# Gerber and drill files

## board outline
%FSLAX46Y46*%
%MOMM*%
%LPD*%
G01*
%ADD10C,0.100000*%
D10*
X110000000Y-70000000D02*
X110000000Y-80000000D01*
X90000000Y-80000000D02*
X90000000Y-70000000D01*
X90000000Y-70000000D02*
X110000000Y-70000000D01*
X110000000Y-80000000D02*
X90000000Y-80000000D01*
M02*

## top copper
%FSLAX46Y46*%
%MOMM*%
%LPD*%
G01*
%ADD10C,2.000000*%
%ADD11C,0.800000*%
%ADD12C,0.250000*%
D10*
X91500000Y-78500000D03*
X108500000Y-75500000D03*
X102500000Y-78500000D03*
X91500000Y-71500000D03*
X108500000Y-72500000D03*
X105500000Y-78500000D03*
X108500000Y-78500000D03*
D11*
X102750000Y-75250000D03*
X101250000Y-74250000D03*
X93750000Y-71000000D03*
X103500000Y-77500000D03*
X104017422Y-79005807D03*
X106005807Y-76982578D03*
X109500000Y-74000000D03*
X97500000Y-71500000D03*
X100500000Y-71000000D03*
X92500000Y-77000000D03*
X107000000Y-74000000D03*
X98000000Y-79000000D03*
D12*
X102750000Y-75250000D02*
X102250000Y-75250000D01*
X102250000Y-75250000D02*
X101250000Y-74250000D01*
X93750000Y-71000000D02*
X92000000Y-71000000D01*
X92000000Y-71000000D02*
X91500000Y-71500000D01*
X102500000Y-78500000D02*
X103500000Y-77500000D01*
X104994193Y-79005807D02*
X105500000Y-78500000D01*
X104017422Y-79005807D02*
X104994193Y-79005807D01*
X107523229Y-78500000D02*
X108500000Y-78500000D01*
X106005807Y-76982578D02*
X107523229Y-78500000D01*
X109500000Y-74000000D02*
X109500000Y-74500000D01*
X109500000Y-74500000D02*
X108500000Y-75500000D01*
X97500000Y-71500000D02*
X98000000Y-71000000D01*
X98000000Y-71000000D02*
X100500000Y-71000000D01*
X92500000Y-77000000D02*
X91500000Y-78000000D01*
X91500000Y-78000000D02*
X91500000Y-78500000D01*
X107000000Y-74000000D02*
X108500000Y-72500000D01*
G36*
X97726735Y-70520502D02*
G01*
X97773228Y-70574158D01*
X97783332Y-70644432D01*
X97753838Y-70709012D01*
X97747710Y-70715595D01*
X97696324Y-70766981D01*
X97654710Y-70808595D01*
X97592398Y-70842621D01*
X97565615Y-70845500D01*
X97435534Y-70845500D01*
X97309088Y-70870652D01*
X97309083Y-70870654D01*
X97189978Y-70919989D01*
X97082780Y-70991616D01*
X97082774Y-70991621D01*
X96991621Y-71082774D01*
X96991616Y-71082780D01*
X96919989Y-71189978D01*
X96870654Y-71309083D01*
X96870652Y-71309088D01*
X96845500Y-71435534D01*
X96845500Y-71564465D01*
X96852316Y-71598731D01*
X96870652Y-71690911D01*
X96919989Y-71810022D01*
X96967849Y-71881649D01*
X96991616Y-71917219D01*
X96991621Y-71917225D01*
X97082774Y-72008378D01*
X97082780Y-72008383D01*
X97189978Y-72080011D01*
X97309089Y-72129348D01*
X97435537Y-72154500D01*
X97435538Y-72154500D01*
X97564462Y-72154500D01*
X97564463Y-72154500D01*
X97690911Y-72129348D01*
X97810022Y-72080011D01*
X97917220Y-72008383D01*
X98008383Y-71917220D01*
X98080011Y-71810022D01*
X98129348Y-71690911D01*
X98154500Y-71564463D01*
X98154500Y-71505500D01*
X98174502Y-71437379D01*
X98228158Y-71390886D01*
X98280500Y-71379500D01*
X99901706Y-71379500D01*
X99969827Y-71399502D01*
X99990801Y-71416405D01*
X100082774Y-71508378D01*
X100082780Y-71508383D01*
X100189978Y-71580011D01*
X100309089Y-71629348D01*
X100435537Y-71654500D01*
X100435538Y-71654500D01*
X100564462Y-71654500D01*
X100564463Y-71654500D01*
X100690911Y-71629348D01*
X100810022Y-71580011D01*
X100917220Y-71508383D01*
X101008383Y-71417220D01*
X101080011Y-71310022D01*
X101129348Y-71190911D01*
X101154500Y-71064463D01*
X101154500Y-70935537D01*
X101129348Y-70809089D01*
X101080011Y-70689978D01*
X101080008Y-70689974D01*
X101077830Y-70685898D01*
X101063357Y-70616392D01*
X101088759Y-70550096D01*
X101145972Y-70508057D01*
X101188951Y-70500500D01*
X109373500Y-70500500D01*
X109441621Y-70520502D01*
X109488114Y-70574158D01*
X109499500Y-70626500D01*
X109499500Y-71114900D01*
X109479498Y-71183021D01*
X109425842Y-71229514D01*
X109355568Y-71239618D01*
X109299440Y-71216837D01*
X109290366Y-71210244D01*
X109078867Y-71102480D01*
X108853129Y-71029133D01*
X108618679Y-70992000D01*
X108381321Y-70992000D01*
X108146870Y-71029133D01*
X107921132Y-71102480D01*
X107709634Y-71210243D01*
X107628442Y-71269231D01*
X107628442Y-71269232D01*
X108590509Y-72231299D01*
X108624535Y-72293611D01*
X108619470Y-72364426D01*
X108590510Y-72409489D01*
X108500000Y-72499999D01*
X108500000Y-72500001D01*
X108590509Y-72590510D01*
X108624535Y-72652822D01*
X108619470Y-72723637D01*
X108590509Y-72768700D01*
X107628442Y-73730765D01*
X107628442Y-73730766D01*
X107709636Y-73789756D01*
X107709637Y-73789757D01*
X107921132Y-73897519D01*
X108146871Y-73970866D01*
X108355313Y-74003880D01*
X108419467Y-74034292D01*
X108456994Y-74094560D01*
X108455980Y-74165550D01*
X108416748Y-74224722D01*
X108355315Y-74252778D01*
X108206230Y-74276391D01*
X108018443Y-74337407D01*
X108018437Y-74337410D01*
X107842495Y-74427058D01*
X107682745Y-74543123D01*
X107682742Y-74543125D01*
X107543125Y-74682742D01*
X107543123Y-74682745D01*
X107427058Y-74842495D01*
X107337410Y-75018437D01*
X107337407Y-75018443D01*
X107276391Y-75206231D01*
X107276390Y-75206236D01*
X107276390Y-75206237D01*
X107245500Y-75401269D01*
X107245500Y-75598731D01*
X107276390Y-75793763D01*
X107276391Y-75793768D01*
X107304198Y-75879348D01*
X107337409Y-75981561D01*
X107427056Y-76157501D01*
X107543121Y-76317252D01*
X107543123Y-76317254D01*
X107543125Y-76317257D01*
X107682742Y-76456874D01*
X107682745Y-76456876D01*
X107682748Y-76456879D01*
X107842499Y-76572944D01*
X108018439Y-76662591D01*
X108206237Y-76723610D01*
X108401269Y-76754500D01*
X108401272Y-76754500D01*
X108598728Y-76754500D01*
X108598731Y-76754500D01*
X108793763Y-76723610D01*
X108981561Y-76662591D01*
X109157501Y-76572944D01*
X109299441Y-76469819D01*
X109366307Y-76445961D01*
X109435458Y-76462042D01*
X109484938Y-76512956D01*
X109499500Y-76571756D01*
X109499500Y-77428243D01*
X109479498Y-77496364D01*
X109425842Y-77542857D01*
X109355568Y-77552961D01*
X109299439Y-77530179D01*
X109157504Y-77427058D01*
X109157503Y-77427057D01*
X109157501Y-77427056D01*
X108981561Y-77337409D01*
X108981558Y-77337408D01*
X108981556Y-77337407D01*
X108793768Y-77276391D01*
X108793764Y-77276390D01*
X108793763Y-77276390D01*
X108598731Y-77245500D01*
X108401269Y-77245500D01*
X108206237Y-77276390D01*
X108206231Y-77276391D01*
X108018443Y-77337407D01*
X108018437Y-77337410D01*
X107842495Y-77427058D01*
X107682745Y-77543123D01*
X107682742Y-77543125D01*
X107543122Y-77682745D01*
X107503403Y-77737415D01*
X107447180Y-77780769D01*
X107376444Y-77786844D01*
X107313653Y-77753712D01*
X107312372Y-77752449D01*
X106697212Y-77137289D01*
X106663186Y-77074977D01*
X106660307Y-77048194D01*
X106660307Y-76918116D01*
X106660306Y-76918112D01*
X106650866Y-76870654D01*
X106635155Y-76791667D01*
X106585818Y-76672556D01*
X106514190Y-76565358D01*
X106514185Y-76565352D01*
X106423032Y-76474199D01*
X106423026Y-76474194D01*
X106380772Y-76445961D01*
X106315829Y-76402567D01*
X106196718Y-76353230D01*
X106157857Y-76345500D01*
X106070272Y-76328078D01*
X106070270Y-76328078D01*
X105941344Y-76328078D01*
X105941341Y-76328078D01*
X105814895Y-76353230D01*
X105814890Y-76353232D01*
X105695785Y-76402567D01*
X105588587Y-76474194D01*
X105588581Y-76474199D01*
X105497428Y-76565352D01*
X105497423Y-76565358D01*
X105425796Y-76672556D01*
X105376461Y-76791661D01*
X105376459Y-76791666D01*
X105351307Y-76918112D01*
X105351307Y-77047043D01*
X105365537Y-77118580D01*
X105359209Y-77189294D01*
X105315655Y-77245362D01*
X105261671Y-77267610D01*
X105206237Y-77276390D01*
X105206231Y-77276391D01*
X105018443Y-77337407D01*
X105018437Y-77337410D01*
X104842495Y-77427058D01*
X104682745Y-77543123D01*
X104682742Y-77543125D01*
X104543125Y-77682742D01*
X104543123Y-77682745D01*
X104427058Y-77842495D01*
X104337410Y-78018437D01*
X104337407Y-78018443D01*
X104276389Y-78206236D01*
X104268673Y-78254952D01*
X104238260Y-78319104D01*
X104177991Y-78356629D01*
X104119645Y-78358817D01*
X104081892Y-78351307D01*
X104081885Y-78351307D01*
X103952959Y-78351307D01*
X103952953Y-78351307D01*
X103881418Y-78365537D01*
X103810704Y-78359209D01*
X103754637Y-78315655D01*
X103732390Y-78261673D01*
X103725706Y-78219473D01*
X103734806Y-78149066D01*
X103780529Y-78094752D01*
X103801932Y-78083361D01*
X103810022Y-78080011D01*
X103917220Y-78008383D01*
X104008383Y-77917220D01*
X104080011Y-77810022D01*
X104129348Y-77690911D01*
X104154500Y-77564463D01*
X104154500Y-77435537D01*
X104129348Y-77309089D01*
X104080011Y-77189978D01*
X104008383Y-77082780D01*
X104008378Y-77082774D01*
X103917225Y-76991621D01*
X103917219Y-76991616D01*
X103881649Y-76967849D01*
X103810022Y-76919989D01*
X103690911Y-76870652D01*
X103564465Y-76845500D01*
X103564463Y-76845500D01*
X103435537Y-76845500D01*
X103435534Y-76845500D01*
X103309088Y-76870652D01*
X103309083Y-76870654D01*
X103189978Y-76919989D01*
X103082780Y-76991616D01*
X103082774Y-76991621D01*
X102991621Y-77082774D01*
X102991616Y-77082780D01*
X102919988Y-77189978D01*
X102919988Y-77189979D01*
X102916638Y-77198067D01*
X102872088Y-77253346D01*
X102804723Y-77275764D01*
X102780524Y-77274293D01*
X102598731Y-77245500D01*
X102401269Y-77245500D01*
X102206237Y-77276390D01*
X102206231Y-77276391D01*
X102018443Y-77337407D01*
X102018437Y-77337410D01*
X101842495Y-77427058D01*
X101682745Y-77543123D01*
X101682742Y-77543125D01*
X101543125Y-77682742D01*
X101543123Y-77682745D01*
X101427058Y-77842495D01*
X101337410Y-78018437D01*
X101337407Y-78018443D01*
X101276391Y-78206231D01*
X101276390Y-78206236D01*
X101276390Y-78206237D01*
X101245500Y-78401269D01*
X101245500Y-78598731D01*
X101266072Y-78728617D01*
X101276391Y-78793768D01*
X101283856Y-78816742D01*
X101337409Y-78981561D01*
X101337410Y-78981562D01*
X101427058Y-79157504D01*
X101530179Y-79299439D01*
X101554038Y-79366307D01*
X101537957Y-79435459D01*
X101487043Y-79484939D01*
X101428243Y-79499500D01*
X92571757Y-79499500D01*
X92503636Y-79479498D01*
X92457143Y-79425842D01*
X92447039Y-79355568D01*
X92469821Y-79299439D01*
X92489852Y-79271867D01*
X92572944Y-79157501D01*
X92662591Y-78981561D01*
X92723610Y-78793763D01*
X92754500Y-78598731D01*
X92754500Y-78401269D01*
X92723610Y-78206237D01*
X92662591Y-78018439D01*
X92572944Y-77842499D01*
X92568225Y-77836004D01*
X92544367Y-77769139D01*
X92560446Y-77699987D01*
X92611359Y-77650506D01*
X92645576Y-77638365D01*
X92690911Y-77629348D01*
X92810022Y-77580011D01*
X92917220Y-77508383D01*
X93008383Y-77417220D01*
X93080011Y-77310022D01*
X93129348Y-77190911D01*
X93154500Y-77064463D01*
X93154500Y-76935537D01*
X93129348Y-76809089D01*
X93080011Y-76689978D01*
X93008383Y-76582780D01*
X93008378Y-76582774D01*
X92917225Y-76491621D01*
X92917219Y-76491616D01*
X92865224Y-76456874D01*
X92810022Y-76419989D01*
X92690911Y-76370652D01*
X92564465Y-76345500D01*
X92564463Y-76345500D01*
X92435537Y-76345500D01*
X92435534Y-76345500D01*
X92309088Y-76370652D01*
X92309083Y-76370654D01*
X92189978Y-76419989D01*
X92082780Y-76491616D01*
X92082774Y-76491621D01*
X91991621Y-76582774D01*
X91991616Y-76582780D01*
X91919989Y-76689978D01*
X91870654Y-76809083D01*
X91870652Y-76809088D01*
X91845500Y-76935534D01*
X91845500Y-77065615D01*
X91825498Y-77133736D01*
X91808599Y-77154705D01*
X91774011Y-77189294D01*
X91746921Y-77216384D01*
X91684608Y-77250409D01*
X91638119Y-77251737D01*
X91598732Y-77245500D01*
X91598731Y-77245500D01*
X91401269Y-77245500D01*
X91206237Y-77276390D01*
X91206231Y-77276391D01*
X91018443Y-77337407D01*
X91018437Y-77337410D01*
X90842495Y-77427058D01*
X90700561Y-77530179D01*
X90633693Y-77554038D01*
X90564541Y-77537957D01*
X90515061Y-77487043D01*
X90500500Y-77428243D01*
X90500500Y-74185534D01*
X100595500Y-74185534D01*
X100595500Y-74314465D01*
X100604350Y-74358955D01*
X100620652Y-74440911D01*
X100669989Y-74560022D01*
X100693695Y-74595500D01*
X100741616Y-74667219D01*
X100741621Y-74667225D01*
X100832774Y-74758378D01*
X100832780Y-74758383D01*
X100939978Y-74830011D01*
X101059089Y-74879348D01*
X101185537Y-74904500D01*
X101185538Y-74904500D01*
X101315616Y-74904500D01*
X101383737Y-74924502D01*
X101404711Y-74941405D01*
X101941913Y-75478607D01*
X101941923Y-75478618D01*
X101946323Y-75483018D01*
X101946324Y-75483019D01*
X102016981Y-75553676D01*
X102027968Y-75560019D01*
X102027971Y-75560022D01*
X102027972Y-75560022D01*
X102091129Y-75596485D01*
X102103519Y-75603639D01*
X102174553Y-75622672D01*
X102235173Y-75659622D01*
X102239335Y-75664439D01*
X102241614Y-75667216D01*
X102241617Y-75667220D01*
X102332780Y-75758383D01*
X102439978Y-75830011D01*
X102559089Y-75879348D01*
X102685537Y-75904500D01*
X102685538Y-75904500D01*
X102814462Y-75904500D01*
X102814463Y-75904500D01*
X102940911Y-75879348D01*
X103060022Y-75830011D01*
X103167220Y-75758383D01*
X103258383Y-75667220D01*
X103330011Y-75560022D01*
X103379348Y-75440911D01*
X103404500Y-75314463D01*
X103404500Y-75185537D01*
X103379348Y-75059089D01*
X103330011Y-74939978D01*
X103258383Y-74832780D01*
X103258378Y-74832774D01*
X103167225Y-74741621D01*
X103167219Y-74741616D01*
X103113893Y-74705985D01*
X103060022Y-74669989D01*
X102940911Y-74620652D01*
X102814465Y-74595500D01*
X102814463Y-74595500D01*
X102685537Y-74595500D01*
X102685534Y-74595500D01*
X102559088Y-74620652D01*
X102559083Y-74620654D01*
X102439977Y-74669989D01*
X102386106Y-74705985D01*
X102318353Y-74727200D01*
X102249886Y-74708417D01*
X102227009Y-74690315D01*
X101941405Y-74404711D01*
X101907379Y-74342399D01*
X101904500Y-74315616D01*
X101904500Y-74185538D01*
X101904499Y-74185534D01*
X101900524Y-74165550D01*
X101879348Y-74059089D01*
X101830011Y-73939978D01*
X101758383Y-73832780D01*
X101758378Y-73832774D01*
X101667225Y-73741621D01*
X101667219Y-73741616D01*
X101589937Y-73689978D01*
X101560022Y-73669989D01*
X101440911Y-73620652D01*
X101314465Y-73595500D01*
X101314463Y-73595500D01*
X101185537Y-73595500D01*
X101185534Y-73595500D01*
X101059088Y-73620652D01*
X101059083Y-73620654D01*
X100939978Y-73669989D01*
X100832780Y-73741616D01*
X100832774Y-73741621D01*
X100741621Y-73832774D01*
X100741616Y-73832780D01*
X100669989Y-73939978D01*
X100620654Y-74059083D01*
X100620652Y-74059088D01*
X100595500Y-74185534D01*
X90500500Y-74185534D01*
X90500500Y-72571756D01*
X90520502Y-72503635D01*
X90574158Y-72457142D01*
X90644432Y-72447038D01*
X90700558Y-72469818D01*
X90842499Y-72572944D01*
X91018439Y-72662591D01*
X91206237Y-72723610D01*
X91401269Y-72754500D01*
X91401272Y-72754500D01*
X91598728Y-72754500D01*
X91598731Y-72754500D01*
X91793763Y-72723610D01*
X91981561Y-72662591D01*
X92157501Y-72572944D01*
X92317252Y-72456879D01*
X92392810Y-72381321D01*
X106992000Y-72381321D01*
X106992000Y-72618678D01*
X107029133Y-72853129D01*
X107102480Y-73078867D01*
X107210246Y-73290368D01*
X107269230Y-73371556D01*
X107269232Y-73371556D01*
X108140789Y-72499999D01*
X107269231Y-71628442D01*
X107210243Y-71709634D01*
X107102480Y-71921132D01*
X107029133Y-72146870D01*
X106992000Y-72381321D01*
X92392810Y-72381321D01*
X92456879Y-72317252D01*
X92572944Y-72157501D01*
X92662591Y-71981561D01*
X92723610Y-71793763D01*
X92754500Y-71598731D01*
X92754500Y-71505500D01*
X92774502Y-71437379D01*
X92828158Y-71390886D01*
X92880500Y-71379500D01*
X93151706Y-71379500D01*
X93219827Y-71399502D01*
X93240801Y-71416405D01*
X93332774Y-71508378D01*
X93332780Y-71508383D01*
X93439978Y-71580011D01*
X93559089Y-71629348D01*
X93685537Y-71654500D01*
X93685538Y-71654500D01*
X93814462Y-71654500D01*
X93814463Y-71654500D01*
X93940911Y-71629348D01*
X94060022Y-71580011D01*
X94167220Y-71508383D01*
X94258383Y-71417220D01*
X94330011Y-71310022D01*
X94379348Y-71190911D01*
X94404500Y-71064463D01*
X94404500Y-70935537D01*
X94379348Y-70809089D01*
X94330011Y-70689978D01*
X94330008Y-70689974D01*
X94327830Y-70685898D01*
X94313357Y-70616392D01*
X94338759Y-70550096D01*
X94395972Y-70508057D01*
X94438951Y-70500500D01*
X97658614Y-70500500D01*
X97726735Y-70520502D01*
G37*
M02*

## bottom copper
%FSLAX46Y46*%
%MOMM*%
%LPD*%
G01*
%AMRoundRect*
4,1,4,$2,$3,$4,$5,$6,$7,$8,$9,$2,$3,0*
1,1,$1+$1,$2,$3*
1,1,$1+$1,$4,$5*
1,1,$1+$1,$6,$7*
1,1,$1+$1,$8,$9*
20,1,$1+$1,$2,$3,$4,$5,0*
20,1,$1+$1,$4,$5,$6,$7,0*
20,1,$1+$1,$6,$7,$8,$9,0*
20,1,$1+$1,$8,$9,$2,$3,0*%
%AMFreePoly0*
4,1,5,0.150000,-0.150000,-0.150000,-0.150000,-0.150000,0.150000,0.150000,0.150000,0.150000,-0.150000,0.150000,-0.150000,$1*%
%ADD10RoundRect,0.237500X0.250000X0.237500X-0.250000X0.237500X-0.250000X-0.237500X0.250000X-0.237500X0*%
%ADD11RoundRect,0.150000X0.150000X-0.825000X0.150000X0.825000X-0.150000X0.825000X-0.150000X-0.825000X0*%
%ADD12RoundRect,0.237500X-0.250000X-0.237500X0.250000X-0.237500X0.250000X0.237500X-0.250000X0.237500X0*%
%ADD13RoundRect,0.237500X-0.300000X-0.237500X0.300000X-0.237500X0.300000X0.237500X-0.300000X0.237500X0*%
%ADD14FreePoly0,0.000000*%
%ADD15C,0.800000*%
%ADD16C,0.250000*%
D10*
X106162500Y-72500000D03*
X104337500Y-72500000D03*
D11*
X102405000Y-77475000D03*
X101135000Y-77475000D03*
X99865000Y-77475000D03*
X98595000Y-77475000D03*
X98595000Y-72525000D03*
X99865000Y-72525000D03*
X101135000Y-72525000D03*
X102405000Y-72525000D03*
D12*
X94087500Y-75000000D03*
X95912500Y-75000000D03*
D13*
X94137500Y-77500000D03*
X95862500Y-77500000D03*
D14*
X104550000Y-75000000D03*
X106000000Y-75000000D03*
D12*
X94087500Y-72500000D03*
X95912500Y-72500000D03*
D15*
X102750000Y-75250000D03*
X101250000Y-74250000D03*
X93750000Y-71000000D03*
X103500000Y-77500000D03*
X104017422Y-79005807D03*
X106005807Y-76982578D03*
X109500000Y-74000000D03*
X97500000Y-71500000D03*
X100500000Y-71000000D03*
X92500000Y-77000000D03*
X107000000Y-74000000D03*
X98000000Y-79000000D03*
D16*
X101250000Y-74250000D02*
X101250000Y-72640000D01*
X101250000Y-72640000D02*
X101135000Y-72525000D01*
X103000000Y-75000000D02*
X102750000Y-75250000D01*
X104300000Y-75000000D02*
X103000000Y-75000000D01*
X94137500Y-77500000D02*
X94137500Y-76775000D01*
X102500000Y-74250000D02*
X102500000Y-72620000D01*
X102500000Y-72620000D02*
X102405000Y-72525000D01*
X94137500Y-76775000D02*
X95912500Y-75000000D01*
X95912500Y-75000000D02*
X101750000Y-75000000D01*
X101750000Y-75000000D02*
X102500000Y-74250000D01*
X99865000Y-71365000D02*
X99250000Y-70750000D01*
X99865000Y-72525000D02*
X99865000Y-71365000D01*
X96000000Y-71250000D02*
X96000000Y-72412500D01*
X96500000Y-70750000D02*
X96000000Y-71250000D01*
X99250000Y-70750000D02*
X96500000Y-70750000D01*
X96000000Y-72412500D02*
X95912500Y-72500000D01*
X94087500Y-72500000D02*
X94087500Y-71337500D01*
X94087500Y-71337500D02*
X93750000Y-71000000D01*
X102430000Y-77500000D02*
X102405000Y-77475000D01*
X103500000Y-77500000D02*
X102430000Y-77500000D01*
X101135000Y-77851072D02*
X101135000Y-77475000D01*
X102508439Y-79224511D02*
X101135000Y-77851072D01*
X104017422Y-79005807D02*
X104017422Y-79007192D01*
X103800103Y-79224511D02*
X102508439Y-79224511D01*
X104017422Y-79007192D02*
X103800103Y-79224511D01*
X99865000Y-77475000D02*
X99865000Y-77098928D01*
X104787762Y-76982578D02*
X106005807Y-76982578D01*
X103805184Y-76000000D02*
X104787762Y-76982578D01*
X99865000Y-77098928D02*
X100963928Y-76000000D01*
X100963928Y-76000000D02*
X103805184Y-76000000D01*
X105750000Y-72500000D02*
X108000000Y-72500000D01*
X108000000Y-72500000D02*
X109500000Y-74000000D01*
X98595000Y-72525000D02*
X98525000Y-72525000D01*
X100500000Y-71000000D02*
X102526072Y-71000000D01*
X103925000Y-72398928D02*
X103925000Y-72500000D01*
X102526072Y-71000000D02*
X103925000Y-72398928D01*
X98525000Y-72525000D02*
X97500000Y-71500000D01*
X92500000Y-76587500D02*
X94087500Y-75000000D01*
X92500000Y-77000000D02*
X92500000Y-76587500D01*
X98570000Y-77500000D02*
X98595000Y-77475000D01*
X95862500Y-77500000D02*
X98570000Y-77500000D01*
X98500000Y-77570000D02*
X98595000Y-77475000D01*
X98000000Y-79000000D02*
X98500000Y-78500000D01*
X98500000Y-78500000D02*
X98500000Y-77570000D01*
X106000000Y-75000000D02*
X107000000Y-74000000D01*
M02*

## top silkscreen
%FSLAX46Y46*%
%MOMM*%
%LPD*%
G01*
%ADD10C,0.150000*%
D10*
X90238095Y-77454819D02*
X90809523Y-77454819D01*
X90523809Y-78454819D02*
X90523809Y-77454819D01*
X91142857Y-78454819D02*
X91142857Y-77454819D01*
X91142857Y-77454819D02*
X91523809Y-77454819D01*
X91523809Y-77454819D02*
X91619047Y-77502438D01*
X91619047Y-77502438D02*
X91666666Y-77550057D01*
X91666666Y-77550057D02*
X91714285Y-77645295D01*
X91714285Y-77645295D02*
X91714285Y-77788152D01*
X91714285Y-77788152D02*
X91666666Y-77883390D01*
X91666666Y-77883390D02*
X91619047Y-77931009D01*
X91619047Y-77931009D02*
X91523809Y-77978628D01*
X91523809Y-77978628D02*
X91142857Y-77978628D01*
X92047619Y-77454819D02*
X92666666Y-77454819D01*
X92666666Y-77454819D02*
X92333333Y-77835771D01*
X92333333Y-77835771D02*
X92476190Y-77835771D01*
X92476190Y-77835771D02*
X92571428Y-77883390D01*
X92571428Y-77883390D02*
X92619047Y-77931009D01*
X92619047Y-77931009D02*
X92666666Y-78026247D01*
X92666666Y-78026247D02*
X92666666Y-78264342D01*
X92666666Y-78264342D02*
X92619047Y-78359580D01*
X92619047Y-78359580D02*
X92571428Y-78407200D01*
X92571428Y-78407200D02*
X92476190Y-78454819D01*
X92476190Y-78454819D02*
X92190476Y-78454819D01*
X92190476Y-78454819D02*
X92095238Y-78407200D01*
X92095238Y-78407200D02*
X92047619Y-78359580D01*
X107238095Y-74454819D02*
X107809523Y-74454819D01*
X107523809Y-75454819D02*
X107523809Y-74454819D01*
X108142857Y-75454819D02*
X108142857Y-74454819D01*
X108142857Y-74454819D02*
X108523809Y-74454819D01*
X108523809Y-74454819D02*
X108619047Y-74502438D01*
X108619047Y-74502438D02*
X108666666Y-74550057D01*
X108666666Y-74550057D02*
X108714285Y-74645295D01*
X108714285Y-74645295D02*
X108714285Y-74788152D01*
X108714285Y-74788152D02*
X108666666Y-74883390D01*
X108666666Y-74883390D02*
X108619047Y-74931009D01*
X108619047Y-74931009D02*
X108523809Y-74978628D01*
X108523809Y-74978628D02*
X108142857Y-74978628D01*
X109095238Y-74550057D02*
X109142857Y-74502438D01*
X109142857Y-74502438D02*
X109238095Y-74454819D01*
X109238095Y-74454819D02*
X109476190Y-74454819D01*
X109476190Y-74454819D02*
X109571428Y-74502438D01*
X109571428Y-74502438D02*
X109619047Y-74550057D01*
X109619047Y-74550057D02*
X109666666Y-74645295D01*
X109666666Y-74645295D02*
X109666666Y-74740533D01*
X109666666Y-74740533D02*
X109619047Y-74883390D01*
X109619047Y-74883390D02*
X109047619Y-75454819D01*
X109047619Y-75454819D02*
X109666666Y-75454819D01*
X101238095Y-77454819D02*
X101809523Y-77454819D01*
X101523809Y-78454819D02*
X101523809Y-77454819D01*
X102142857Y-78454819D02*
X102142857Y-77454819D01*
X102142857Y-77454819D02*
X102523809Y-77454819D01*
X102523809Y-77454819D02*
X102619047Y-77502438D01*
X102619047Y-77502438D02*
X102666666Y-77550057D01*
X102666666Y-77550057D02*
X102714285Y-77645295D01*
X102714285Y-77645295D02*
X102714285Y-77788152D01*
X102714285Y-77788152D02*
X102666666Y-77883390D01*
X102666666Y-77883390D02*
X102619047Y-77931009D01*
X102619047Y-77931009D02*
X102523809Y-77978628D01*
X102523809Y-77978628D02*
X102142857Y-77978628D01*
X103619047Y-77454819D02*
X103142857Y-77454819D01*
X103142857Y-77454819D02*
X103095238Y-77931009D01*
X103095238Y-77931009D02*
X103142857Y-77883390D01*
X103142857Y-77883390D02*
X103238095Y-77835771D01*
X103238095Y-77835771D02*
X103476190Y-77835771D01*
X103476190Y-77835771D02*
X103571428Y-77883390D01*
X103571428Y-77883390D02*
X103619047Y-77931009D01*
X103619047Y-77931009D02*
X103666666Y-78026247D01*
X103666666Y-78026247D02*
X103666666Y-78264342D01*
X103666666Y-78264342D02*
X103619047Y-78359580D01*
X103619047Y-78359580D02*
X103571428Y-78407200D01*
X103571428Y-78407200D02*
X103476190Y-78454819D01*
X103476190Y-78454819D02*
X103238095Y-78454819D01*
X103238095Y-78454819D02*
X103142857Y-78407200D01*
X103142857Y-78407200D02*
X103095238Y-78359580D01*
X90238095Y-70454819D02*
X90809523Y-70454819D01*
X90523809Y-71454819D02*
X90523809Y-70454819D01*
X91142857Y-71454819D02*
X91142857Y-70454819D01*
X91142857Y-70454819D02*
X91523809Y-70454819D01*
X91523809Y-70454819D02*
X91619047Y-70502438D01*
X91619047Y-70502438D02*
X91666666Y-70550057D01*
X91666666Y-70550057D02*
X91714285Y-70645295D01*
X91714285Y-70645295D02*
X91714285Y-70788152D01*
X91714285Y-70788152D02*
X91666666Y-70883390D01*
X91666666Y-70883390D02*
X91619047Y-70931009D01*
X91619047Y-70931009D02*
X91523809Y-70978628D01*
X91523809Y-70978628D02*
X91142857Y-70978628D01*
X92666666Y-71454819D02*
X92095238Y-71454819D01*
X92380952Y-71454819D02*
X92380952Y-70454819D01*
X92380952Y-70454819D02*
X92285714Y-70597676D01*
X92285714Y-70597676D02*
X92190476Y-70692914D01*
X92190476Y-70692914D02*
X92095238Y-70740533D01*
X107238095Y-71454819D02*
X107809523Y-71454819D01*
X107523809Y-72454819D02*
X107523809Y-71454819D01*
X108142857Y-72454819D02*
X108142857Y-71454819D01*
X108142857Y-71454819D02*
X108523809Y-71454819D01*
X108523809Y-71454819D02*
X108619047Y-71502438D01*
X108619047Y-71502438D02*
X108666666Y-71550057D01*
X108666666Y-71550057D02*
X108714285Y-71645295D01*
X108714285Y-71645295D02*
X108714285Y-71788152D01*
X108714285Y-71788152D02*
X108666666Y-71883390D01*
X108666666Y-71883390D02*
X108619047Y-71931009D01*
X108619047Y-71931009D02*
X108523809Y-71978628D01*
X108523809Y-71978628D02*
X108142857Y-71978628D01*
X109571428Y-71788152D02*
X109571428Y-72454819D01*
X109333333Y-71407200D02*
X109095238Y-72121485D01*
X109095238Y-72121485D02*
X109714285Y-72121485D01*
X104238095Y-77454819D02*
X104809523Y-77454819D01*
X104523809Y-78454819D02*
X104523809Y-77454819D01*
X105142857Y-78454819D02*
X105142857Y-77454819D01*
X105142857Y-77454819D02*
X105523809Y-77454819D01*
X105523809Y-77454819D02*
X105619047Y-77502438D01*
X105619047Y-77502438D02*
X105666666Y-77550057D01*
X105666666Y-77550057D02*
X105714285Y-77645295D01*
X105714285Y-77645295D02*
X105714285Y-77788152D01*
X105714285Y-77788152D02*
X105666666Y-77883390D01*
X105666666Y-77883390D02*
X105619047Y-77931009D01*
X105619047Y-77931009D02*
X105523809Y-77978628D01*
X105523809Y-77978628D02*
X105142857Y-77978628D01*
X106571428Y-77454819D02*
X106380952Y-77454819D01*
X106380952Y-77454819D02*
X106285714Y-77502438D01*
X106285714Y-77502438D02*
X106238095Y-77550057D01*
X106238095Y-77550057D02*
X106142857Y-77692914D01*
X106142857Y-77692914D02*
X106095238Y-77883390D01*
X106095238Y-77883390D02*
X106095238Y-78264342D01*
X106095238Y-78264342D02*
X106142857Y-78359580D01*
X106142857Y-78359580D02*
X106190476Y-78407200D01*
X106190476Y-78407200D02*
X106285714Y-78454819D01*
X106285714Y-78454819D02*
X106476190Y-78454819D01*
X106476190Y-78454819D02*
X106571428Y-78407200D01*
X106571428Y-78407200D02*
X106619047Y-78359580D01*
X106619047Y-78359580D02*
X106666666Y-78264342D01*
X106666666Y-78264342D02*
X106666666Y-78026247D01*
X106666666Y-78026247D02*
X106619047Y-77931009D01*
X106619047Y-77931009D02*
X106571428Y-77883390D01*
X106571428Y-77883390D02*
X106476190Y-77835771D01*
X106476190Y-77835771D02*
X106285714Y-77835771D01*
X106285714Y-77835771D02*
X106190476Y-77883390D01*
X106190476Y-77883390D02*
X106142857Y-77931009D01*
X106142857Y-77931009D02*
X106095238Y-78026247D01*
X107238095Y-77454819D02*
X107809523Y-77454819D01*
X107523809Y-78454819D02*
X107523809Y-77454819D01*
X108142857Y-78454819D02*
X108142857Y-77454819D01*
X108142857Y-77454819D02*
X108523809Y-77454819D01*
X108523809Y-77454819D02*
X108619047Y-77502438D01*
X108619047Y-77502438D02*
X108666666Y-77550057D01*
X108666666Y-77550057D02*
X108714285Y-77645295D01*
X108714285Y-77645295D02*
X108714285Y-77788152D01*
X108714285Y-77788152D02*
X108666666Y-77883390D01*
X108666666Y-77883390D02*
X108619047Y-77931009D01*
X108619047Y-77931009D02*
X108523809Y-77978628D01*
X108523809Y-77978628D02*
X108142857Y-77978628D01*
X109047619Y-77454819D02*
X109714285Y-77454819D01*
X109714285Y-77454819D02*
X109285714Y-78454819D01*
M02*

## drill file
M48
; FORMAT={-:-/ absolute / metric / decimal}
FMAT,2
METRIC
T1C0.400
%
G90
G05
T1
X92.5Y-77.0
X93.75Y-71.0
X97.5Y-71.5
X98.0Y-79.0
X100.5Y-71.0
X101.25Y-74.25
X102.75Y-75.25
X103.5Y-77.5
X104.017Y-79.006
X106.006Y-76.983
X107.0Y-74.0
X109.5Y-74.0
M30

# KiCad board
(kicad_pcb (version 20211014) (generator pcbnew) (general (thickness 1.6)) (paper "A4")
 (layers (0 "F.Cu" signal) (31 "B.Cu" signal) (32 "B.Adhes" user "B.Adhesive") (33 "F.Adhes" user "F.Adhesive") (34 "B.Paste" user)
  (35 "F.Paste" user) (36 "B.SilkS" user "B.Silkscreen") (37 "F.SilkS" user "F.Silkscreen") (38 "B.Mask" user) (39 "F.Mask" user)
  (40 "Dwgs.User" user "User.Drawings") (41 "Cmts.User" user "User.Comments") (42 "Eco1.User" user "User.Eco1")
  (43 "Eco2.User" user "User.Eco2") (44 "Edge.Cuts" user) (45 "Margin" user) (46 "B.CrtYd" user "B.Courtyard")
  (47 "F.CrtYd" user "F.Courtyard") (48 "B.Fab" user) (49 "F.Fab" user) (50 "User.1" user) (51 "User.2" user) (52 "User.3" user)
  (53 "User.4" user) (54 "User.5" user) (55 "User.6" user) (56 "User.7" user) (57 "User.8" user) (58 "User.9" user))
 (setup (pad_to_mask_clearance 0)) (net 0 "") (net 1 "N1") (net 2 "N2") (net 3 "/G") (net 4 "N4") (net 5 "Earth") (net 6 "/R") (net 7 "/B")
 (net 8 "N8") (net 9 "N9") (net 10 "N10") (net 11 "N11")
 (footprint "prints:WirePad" (layer "F.Cu") (at 91.5 78.5)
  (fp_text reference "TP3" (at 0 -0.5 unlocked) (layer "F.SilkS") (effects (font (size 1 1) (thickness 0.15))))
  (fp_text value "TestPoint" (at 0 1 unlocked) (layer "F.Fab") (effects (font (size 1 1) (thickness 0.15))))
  (pad "1" smd circle (at 0 0) (size 2 2) (layers "F.Cu" "F.Paste" "F.Mask") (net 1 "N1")))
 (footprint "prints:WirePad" (layer "F.Cu") (at 108.5 75.5)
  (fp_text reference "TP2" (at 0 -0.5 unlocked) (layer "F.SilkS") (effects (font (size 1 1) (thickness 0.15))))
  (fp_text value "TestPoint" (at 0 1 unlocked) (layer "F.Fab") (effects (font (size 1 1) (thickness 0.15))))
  (pad "1" smd circle (at 0 0) (size 2 2) (layers "F.Cu" "F.Paste" "F.Mask") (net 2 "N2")))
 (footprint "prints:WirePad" (layer "F.Cu") (at 102.5 78.5)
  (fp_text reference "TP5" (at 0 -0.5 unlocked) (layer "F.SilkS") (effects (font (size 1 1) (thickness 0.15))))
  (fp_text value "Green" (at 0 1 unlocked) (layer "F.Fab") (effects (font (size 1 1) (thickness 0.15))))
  (pad "1" smd circle (at 0 0) (size 2 2) (layers "F.Cu" "F.Paste" "F.Mask") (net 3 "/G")))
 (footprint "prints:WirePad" (layer "F.Cu") (at 91.5 71.5)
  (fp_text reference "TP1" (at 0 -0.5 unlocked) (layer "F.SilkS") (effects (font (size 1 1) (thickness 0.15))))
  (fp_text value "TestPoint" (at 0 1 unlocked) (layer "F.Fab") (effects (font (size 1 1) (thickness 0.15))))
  (pad "1" smd circle (at 0 0) (size 2 2) (layers "F.Cu" "F.Paste" "F.Mask") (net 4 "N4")))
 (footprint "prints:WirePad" (layer "F.Cu") (at 108.5 72.5)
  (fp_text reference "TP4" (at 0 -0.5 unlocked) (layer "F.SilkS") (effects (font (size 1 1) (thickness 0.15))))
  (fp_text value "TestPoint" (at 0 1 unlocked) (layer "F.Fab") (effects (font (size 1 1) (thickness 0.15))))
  (pad "1" smd circle (at 0 0) (size 2 2) (layers "F.Cu" "F.Paste" "F.Mask") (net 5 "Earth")))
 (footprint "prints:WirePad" (layer "F.Cu") (at 105.5 78.5)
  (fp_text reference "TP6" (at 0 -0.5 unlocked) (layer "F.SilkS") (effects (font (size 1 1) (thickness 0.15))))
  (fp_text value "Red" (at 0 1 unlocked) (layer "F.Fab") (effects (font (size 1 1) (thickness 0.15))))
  (pad "1" smd circle (at 0 0) (size 2 2) (layers "F.Cu" "F.Paste" "F.Mask") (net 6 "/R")))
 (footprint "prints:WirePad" (layer "F.Cu") (at 108.5 78.5)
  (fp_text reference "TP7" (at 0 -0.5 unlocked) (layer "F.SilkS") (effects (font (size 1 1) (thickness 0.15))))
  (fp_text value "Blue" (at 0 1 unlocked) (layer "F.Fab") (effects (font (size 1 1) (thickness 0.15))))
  (pad "1" smd circle (at 0 0) (size 2 2) (layers "F.Cu" "F.Paste" "F.Mask") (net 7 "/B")))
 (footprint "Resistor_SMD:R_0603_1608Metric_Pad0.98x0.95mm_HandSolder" (layer "B.Cu") (at 105.25 72.5 180)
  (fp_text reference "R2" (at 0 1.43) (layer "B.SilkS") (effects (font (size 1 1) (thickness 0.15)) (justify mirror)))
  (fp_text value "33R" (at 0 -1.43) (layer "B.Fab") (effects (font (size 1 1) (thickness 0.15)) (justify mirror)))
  (pad "1" smd roundrect locked (at -0.9125 0 180) (size 0.975 0.95) (layers "B.Cu" "B.Paste" "B.Mask") (roundrect_rratio 0.25) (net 2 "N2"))
  (pad "2" smd roundrect locked (at 0.9125 0 180) (size 0.975 0.95) (layers "B.Cu" "B.Paste" "B.Mask") (roundrect_rratio 0.25) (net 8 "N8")))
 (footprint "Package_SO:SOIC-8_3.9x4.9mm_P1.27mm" (layer "B.Cu") (at 100.5 75 90)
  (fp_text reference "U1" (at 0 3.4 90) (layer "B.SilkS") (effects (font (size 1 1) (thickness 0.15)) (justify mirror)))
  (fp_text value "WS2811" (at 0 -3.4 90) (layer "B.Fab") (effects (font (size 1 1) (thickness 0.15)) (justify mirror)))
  (pad "1" smd roundrect locked (at -2.475 1.905 90) (size 1.95 0.6) (layers "B.Cu" "B.Paste" "B.Mask") (roundrect_rratio 0.25) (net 3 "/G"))
  (pad "2" smd roundrect locked (at -2.475 0.635 90) (size 1.95 0.6) (layers "B.Cu" "B.Paste" "B.Mask") (roundrect_rratio 0.25) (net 6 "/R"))
  (pad "3" smd roundrect locked (at -2.475 -0.635 90) (size 1.95 0.6) (layers "B.Cu" "B.Paste" "B.Mask") (roundrect_rratio 0.25)
   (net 7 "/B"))
  (pad "4" smd roundrect locked (at -2.475 -1.905 90) (size 1.95 0.6) (layers "B.Cu" "B.Paste" "B.Mask") (roundrect_rratio 0.25)
   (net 5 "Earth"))
  (pad "5" smd roundrect locked (at 2.475 -1.905 90) (size 1.95 0.6) (layers "B.Cu" "B.Paste" "B.Mask") (roundrect_rratio 0.25) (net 8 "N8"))
  (pad "6" smd roundrect locked (at 2.475 -0.635 90) (size 1.95 0.6) (layers "B.Cu" "B.Paste" "B.Mask") (roundrect_rratio 0.25) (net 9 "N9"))
  (pad "7" smd roundrect locked (at 2.475 0.635 90) (size 1.95 0.6) (layers "B.Cu" "B.Paste" "B.Mask") (roundrect_rratio 0.25)
   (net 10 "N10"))
  (pad "8" smd roundrect locked (at 2.475 1.905 90) (size 1.95 0.6) (layers "B.Cu" "B.Paste" "B.Mask") (roundrect_rratio 0.25)
   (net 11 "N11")))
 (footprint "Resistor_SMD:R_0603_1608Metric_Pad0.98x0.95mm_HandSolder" (layer "B.Cu") (at 95 75)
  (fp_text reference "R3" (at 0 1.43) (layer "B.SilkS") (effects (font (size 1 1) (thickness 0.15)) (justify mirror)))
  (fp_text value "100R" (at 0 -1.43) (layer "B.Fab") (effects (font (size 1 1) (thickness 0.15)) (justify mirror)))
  (pad "1" smd roundrect locked (at -0.9125 0) (size 0.975 0.95) (layers "B.Cu" "B.Paste" "B.Mask") (roundrect_rratio 0.25) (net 1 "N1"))
  (pad "2" smd roundrect locked (at 0.9125 0) (size 0.975 0.95) (layers "B.Cu" "B.Paste" "B.Mask") (roundrect_rratio 0.25) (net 11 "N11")))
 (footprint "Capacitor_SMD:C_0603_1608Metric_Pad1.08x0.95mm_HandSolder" (layer "B.Cu") (at 95 77.5)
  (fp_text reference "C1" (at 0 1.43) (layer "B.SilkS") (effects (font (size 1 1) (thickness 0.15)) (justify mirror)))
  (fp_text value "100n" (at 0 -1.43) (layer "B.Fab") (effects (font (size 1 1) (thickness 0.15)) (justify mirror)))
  (pad "1" smd roundrect locked (at -0.8625 0) (size 1.075 0.95) (layers "B.Cu" "B.Paste" "B.Mask") (roundrect_rratio 0.25) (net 11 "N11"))
  (pad "2" smd roundrect locked (at 0.8625 0) (size 1.075 0.95) (layers "B.Cu" "B.Paste" "B.Mask") (roundrect_rratio 0.25) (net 5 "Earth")))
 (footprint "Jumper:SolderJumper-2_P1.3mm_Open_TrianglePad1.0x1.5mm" (layer "B.Cu") (at 105.275 75)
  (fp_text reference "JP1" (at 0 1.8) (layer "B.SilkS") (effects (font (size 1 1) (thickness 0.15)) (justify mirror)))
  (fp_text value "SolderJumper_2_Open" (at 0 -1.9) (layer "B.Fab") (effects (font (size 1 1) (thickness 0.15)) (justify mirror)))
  (pad "1" smd custom locked (at -0.725 0) (size 0.3 0.3) (layers "B.Cu" "B.Mask") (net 10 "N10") (zone_connect 2)
   (options (clearance outline) (anchor rect)) (primitives))
  (pad "2" smd custom locked (at 0.725 0) (size 0.3 0.3) (layers "B.Cu" "B.Mask") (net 5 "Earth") (zone_connect 2)
   (options (clearance outline) (anchor rect)) (primitives)))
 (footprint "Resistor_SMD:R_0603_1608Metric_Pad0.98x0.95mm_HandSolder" (layer "B.Cu") (at 95 72.5)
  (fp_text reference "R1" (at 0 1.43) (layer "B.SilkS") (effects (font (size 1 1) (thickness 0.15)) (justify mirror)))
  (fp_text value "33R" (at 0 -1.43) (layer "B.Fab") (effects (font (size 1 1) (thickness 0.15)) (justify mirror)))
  (pad "1" smd roundrect locked (at -0.9125 0) (size 0.975 0.95) (layers "B.Cu" "B.Paste" "B.Mask") (roundrect_rratio 0.25) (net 4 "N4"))
  (pad "2" smd roundrect locked (at 0.9125 0) (size 0.975 0.95) (layers "B.Cu" "B.Paste" "B.Mask") (roundrect_rratio 0.25) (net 9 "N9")))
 (gr_line (start 110 70) (end 110 80) (layer "Edge.Cuts") (width 0.1))
 (gr_line (start 90 80) (end 90 70) (layer "Edge.Cuts") (width 0.1))
 (gr_line (start 90 70) (end 110 70) (layer "Edge.Cuts") (width 0.1))
 (gr_line (start 110 80) (end 90 80) (layer "Edge.Cuts") (width 0.1))
 (segment (start 102.75 75.25) (end 102.25 75.25) (width 0.25) (layer "F.Cu") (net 10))
 (segment (start 102.25 75.25) (end 101.25 74.25) (width 0.25) (layer "F.Cu") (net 10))
 (via (at 102.75 75.25) (size 0.8) (drill 0.4) (layers "F.Cu" "B.Cu") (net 10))
 (via (at 101.25 74.25) (size 0.8) (drill 0.4) (layers "F.Cu" "B.Cu") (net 10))
 (segment (start 101.25 74.25) (end 101.25 72.64) (width 0.25) (layer "B.Cu") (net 10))
 (segment (start 101.25 72.64) (end 101.135 72.525) (width 0.25) (layer "B.Cu") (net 10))
 (segment (start 103 75) (end 102.75 75.25) (width 0.25) (layer "B.Cu") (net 10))
 (segment (start 104.3 75) (end 103 75) (width 0.25) (layer "B.Cu") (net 10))
 (segment (start 94.1375 77.5) (end 94.1375 76.775) (width 0.25) (layer "B.Cu") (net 11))
 (segment (start 102.5 74.25) (end 102.5 72.62) (width 0.25) (layer "B.Cu") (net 11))
 (segment (start 102.5 72.62) (end 102.405 72.525) (width 0.25) (layer "B.Cu") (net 11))
 (segment (start 94.1375 76.775) (end 95.9125 75) (width 0.25) (layer "B.Cu") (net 11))
 (segment (start 95.9125 75) (end 101.75 75) (width 0.25) (layer "B.Cu") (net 11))
 (segment (start 101.75 75) (end 102.5 74.25) (width 0.25) (layer "B.Cu") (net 11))
 (segment (start 99.865 71.365) (end 99.25 70.75) (width 0.25) (layer "B.Cu") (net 9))
 (segment (start 99.865 72.525) (end 99.865 71.365) (width 0.25) (layer "B.Cu") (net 9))
 (segment (start 96 71.25) (end 96 72.4125) (width 0.25) (layer "B.Cu") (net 9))
 (segment (start 96.5 70.75) (end 96 71.25) (width 0.25) (layer "B.Cu") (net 9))
 (segment (start 99.25 70.75) (end 96.5 70.75) (width 0.25) (layer "B.Cu") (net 9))
 (segment (start 96 72.4125) (end 95.9125 72.5) (width 0.25) (layer "B.Cu") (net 9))
 (segment (start 93.75 71) (end 92 71) (width 0.25) (layer "F.Cu") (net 4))
 (segment (start 92 71) (end 91.5 71.5) (width 0.25) (layer "F.Cu") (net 4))
 (via (at 93.75 71) (size 0.8) (drill 0.4) (layers "F.Cu" "B.Cu") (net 4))
 (segment (start 94.0875 72.5) (end 94.0875 71.3375) (width 0.25) (layer "B.Cu") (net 4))
 (segment (start 94.0875 71.3375) (end 93.75 71) (width 0.25) (layer "B.Cu") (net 4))
 (segment (start 102.5 78.5) (end 103.5 77.5) (width 0.25) (layer "F.Cu") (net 3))
 (via (at 103.5 77.5) (size 0.8) (drill 0.4) (layers "F.Cu" "B.Cu") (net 3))
 (segment (start 102.43 77.5) (end 102.405 77.475) (width 0.25) (layer "B.Cu") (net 3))
 (segment (start 103.5 77.5) (end 102.43 77.5) (width 0.25) (layer "B.Cu") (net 3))
 (segment (start 104.994193 79.005807) (end 105.5 78.5) (width 0.25) (layer "F.Cu") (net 6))
 (segment (start 104.017422 79.005807) (end 104.994193 79.005807) (width 0.25) (layer "F.Cu") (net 6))
 (via (at 104.017422 79.005807) (size 0.8) (drill 0.4) (layers "F.Cu" "B.Cu") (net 6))
 (segment (start 101.135 77.851072) (end 101.135 77.475) (width 0.25) (layer "B.Cu") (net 6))
 (segment (start 102.508439 79.224511) (end 101.135 77.851072) (width 0.25) (layer "B.Cu") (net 6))
 (segment (start 104.017422 79.005807) (end 104.017422 79.007192) (width 0.25) (layer "B.Cu") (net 6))
 (segment (start 103.800103 79.224511) (end 102.508439 79.224511) (width 0.25) (layer "B.Cu") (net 6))
 (segment (start 104.017422 79.007192) (end 103.800103 79.224511) (width 0.25) (layer "B.Cu") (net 6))
 (segment (start 107.523229 78.5) (end 108.5 78.5) (width 0.25) (layer "F.Cu") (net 7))
 (segment (start 106.005807 76.982578) (end 107.523229 78.5) (width 0.25) (layer "F.Cu") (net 7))
 (via (at 106.005807 76.982578) (size 0.8) (drill 0.4) (layers "F.Cu" "B.Cu") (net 7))
 (segment (start 99.865 77.475) (end 99.865 77.098928) (width 0.25) (layer "B.Cu") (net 7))
 (segment (start 104.787762 76.982578) (end 106.005807 76.982578) (width 0.25) (layer "B.Cu") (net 7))
 (segment (start 103.805184 76) (end 104.787762 76.982578) (width 0.25) (layer "B.Cu") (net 7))
 (segment (start 99.865 77.098928) (end 100.963928 76) (width 0.25) (layer "B.Cu") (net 7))
 (segment (start 100.963928 76) (end 103.805184 76) (width 0.25) (layer "B.Cu") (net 7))
 (segment (start 109.5 74) (end 109.5 74.5) (width 0.25) (layer "F.Cu") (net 2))
 (segment (start 109.5 74.5) (end 108.5 75.5) (width 0.25) (layer "F.Cu") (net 2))
 (via (at 109.5 74) (size 0.8) (drill 0.4) (layers "F.Cu" "B.Cu") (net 2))
 (segment (start 105.75 72.5) (end 108 72.5) (width 0.25) (layer "B.Cu") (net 2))
 (segment (start 108 72.5) (end 109.5 74) (width 0.25) (layer "B.Cu") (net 2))
 (segment (start 97.5 71.5) (end 98 71) (width 0.25) (layer "F.Cu") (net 8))
 (segment (start 98 71) (end 100.5 71) (width 0.25) (layer "F.Cu") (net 8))
 (via (at 97.5 71.5) (size 0.8) (drill 0.4) (layers "F.Cu" "B.Cu") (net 8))
 (via (at 100.5 71) (size 0.8) (drill 0.4) (layers "F.Cu" "B.Cu") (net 8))
 (segment (start 98.595 72.525) (end 98.525 72.525) (width 0.25) (layer "B.Cu") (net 8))
 (segment (start 100.5 71) (end 102.526072 71) (width 0.25) (layer "B.Cu") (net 8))
 (segment (start 103.925 72.398928) (end 103.925 72.5) (width 0.25) (layer "B.Cu") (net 8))
 (segment (start 102.526072 71) (end 103.925 72.398928) (width 0.25) (layer "B.Cu") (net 8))
 (segment (start 98.525 72.525) (end 97.5 71.5) (width 0.25) (layer "B.Cu") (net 8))
 (segment (start 92.5 77) (end 91.5 78) (width 0.25) (layer "F.Cu") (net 1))
 (segment (start 91.5 78) (end 91.5 78.5) (width 0.25) (layer "F.Cu") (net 1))
 (via (at 92.5 77) (size 0.8) (drill 0.4) (layers "F.Cu" "B.Cu") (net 1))
 (segment (start 92.5 76.5875) (end 94.0875 75) (width 0.25) (layer "B.Cu") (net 1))
 (segment (start 92.5 77) (end 92.5 76.5875) (width 0.25) (layer "B.Cu") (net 1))
 (segment (start 107 74) (end 108.5 72.5) (width 0.25) (layer "F.Cu") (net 5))
 (via (at 107 74) (size 0.8) (drill 0.4) (layers "F.Cu" "B.Cu") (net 5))
 (via (at 98 79) (size 0.8) (drill 0.4) (layers "F.Cu" "B.Cu") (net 5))
 (segment (start 98.57 77.5) (end 98.595 77.475) (width 0.25) (layer "B.Cu") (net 5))
 (segment (start 95.8625 77.5) (end 98.57 77.5) (width 0.25) (layer "B.Cu") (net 5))
 (segment (start 98.5 77.57) (end 98.595 77.475) (width 0.25) (layer "B.Cu") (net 5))
 (segment (start 98 79) (end 98.5 78.5) (width 0.25) (layer "B.Cu") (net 5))
 (segment (start 98.5 78.5) (end 98.5 77.57) (width 0.25) (layer "B.Cu") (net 5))
 (segment (start 106 75) (end 107 74) (width 0.25) (layer "B.Cu") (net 5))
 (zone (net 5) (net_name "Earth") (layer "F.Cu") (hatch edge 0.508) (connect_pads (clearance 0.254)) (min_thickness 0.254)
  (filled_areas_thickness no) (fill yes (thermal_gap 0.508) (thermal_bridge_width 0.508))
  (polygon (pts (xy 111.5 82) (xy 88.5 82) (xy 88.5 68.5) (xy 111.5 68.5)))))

